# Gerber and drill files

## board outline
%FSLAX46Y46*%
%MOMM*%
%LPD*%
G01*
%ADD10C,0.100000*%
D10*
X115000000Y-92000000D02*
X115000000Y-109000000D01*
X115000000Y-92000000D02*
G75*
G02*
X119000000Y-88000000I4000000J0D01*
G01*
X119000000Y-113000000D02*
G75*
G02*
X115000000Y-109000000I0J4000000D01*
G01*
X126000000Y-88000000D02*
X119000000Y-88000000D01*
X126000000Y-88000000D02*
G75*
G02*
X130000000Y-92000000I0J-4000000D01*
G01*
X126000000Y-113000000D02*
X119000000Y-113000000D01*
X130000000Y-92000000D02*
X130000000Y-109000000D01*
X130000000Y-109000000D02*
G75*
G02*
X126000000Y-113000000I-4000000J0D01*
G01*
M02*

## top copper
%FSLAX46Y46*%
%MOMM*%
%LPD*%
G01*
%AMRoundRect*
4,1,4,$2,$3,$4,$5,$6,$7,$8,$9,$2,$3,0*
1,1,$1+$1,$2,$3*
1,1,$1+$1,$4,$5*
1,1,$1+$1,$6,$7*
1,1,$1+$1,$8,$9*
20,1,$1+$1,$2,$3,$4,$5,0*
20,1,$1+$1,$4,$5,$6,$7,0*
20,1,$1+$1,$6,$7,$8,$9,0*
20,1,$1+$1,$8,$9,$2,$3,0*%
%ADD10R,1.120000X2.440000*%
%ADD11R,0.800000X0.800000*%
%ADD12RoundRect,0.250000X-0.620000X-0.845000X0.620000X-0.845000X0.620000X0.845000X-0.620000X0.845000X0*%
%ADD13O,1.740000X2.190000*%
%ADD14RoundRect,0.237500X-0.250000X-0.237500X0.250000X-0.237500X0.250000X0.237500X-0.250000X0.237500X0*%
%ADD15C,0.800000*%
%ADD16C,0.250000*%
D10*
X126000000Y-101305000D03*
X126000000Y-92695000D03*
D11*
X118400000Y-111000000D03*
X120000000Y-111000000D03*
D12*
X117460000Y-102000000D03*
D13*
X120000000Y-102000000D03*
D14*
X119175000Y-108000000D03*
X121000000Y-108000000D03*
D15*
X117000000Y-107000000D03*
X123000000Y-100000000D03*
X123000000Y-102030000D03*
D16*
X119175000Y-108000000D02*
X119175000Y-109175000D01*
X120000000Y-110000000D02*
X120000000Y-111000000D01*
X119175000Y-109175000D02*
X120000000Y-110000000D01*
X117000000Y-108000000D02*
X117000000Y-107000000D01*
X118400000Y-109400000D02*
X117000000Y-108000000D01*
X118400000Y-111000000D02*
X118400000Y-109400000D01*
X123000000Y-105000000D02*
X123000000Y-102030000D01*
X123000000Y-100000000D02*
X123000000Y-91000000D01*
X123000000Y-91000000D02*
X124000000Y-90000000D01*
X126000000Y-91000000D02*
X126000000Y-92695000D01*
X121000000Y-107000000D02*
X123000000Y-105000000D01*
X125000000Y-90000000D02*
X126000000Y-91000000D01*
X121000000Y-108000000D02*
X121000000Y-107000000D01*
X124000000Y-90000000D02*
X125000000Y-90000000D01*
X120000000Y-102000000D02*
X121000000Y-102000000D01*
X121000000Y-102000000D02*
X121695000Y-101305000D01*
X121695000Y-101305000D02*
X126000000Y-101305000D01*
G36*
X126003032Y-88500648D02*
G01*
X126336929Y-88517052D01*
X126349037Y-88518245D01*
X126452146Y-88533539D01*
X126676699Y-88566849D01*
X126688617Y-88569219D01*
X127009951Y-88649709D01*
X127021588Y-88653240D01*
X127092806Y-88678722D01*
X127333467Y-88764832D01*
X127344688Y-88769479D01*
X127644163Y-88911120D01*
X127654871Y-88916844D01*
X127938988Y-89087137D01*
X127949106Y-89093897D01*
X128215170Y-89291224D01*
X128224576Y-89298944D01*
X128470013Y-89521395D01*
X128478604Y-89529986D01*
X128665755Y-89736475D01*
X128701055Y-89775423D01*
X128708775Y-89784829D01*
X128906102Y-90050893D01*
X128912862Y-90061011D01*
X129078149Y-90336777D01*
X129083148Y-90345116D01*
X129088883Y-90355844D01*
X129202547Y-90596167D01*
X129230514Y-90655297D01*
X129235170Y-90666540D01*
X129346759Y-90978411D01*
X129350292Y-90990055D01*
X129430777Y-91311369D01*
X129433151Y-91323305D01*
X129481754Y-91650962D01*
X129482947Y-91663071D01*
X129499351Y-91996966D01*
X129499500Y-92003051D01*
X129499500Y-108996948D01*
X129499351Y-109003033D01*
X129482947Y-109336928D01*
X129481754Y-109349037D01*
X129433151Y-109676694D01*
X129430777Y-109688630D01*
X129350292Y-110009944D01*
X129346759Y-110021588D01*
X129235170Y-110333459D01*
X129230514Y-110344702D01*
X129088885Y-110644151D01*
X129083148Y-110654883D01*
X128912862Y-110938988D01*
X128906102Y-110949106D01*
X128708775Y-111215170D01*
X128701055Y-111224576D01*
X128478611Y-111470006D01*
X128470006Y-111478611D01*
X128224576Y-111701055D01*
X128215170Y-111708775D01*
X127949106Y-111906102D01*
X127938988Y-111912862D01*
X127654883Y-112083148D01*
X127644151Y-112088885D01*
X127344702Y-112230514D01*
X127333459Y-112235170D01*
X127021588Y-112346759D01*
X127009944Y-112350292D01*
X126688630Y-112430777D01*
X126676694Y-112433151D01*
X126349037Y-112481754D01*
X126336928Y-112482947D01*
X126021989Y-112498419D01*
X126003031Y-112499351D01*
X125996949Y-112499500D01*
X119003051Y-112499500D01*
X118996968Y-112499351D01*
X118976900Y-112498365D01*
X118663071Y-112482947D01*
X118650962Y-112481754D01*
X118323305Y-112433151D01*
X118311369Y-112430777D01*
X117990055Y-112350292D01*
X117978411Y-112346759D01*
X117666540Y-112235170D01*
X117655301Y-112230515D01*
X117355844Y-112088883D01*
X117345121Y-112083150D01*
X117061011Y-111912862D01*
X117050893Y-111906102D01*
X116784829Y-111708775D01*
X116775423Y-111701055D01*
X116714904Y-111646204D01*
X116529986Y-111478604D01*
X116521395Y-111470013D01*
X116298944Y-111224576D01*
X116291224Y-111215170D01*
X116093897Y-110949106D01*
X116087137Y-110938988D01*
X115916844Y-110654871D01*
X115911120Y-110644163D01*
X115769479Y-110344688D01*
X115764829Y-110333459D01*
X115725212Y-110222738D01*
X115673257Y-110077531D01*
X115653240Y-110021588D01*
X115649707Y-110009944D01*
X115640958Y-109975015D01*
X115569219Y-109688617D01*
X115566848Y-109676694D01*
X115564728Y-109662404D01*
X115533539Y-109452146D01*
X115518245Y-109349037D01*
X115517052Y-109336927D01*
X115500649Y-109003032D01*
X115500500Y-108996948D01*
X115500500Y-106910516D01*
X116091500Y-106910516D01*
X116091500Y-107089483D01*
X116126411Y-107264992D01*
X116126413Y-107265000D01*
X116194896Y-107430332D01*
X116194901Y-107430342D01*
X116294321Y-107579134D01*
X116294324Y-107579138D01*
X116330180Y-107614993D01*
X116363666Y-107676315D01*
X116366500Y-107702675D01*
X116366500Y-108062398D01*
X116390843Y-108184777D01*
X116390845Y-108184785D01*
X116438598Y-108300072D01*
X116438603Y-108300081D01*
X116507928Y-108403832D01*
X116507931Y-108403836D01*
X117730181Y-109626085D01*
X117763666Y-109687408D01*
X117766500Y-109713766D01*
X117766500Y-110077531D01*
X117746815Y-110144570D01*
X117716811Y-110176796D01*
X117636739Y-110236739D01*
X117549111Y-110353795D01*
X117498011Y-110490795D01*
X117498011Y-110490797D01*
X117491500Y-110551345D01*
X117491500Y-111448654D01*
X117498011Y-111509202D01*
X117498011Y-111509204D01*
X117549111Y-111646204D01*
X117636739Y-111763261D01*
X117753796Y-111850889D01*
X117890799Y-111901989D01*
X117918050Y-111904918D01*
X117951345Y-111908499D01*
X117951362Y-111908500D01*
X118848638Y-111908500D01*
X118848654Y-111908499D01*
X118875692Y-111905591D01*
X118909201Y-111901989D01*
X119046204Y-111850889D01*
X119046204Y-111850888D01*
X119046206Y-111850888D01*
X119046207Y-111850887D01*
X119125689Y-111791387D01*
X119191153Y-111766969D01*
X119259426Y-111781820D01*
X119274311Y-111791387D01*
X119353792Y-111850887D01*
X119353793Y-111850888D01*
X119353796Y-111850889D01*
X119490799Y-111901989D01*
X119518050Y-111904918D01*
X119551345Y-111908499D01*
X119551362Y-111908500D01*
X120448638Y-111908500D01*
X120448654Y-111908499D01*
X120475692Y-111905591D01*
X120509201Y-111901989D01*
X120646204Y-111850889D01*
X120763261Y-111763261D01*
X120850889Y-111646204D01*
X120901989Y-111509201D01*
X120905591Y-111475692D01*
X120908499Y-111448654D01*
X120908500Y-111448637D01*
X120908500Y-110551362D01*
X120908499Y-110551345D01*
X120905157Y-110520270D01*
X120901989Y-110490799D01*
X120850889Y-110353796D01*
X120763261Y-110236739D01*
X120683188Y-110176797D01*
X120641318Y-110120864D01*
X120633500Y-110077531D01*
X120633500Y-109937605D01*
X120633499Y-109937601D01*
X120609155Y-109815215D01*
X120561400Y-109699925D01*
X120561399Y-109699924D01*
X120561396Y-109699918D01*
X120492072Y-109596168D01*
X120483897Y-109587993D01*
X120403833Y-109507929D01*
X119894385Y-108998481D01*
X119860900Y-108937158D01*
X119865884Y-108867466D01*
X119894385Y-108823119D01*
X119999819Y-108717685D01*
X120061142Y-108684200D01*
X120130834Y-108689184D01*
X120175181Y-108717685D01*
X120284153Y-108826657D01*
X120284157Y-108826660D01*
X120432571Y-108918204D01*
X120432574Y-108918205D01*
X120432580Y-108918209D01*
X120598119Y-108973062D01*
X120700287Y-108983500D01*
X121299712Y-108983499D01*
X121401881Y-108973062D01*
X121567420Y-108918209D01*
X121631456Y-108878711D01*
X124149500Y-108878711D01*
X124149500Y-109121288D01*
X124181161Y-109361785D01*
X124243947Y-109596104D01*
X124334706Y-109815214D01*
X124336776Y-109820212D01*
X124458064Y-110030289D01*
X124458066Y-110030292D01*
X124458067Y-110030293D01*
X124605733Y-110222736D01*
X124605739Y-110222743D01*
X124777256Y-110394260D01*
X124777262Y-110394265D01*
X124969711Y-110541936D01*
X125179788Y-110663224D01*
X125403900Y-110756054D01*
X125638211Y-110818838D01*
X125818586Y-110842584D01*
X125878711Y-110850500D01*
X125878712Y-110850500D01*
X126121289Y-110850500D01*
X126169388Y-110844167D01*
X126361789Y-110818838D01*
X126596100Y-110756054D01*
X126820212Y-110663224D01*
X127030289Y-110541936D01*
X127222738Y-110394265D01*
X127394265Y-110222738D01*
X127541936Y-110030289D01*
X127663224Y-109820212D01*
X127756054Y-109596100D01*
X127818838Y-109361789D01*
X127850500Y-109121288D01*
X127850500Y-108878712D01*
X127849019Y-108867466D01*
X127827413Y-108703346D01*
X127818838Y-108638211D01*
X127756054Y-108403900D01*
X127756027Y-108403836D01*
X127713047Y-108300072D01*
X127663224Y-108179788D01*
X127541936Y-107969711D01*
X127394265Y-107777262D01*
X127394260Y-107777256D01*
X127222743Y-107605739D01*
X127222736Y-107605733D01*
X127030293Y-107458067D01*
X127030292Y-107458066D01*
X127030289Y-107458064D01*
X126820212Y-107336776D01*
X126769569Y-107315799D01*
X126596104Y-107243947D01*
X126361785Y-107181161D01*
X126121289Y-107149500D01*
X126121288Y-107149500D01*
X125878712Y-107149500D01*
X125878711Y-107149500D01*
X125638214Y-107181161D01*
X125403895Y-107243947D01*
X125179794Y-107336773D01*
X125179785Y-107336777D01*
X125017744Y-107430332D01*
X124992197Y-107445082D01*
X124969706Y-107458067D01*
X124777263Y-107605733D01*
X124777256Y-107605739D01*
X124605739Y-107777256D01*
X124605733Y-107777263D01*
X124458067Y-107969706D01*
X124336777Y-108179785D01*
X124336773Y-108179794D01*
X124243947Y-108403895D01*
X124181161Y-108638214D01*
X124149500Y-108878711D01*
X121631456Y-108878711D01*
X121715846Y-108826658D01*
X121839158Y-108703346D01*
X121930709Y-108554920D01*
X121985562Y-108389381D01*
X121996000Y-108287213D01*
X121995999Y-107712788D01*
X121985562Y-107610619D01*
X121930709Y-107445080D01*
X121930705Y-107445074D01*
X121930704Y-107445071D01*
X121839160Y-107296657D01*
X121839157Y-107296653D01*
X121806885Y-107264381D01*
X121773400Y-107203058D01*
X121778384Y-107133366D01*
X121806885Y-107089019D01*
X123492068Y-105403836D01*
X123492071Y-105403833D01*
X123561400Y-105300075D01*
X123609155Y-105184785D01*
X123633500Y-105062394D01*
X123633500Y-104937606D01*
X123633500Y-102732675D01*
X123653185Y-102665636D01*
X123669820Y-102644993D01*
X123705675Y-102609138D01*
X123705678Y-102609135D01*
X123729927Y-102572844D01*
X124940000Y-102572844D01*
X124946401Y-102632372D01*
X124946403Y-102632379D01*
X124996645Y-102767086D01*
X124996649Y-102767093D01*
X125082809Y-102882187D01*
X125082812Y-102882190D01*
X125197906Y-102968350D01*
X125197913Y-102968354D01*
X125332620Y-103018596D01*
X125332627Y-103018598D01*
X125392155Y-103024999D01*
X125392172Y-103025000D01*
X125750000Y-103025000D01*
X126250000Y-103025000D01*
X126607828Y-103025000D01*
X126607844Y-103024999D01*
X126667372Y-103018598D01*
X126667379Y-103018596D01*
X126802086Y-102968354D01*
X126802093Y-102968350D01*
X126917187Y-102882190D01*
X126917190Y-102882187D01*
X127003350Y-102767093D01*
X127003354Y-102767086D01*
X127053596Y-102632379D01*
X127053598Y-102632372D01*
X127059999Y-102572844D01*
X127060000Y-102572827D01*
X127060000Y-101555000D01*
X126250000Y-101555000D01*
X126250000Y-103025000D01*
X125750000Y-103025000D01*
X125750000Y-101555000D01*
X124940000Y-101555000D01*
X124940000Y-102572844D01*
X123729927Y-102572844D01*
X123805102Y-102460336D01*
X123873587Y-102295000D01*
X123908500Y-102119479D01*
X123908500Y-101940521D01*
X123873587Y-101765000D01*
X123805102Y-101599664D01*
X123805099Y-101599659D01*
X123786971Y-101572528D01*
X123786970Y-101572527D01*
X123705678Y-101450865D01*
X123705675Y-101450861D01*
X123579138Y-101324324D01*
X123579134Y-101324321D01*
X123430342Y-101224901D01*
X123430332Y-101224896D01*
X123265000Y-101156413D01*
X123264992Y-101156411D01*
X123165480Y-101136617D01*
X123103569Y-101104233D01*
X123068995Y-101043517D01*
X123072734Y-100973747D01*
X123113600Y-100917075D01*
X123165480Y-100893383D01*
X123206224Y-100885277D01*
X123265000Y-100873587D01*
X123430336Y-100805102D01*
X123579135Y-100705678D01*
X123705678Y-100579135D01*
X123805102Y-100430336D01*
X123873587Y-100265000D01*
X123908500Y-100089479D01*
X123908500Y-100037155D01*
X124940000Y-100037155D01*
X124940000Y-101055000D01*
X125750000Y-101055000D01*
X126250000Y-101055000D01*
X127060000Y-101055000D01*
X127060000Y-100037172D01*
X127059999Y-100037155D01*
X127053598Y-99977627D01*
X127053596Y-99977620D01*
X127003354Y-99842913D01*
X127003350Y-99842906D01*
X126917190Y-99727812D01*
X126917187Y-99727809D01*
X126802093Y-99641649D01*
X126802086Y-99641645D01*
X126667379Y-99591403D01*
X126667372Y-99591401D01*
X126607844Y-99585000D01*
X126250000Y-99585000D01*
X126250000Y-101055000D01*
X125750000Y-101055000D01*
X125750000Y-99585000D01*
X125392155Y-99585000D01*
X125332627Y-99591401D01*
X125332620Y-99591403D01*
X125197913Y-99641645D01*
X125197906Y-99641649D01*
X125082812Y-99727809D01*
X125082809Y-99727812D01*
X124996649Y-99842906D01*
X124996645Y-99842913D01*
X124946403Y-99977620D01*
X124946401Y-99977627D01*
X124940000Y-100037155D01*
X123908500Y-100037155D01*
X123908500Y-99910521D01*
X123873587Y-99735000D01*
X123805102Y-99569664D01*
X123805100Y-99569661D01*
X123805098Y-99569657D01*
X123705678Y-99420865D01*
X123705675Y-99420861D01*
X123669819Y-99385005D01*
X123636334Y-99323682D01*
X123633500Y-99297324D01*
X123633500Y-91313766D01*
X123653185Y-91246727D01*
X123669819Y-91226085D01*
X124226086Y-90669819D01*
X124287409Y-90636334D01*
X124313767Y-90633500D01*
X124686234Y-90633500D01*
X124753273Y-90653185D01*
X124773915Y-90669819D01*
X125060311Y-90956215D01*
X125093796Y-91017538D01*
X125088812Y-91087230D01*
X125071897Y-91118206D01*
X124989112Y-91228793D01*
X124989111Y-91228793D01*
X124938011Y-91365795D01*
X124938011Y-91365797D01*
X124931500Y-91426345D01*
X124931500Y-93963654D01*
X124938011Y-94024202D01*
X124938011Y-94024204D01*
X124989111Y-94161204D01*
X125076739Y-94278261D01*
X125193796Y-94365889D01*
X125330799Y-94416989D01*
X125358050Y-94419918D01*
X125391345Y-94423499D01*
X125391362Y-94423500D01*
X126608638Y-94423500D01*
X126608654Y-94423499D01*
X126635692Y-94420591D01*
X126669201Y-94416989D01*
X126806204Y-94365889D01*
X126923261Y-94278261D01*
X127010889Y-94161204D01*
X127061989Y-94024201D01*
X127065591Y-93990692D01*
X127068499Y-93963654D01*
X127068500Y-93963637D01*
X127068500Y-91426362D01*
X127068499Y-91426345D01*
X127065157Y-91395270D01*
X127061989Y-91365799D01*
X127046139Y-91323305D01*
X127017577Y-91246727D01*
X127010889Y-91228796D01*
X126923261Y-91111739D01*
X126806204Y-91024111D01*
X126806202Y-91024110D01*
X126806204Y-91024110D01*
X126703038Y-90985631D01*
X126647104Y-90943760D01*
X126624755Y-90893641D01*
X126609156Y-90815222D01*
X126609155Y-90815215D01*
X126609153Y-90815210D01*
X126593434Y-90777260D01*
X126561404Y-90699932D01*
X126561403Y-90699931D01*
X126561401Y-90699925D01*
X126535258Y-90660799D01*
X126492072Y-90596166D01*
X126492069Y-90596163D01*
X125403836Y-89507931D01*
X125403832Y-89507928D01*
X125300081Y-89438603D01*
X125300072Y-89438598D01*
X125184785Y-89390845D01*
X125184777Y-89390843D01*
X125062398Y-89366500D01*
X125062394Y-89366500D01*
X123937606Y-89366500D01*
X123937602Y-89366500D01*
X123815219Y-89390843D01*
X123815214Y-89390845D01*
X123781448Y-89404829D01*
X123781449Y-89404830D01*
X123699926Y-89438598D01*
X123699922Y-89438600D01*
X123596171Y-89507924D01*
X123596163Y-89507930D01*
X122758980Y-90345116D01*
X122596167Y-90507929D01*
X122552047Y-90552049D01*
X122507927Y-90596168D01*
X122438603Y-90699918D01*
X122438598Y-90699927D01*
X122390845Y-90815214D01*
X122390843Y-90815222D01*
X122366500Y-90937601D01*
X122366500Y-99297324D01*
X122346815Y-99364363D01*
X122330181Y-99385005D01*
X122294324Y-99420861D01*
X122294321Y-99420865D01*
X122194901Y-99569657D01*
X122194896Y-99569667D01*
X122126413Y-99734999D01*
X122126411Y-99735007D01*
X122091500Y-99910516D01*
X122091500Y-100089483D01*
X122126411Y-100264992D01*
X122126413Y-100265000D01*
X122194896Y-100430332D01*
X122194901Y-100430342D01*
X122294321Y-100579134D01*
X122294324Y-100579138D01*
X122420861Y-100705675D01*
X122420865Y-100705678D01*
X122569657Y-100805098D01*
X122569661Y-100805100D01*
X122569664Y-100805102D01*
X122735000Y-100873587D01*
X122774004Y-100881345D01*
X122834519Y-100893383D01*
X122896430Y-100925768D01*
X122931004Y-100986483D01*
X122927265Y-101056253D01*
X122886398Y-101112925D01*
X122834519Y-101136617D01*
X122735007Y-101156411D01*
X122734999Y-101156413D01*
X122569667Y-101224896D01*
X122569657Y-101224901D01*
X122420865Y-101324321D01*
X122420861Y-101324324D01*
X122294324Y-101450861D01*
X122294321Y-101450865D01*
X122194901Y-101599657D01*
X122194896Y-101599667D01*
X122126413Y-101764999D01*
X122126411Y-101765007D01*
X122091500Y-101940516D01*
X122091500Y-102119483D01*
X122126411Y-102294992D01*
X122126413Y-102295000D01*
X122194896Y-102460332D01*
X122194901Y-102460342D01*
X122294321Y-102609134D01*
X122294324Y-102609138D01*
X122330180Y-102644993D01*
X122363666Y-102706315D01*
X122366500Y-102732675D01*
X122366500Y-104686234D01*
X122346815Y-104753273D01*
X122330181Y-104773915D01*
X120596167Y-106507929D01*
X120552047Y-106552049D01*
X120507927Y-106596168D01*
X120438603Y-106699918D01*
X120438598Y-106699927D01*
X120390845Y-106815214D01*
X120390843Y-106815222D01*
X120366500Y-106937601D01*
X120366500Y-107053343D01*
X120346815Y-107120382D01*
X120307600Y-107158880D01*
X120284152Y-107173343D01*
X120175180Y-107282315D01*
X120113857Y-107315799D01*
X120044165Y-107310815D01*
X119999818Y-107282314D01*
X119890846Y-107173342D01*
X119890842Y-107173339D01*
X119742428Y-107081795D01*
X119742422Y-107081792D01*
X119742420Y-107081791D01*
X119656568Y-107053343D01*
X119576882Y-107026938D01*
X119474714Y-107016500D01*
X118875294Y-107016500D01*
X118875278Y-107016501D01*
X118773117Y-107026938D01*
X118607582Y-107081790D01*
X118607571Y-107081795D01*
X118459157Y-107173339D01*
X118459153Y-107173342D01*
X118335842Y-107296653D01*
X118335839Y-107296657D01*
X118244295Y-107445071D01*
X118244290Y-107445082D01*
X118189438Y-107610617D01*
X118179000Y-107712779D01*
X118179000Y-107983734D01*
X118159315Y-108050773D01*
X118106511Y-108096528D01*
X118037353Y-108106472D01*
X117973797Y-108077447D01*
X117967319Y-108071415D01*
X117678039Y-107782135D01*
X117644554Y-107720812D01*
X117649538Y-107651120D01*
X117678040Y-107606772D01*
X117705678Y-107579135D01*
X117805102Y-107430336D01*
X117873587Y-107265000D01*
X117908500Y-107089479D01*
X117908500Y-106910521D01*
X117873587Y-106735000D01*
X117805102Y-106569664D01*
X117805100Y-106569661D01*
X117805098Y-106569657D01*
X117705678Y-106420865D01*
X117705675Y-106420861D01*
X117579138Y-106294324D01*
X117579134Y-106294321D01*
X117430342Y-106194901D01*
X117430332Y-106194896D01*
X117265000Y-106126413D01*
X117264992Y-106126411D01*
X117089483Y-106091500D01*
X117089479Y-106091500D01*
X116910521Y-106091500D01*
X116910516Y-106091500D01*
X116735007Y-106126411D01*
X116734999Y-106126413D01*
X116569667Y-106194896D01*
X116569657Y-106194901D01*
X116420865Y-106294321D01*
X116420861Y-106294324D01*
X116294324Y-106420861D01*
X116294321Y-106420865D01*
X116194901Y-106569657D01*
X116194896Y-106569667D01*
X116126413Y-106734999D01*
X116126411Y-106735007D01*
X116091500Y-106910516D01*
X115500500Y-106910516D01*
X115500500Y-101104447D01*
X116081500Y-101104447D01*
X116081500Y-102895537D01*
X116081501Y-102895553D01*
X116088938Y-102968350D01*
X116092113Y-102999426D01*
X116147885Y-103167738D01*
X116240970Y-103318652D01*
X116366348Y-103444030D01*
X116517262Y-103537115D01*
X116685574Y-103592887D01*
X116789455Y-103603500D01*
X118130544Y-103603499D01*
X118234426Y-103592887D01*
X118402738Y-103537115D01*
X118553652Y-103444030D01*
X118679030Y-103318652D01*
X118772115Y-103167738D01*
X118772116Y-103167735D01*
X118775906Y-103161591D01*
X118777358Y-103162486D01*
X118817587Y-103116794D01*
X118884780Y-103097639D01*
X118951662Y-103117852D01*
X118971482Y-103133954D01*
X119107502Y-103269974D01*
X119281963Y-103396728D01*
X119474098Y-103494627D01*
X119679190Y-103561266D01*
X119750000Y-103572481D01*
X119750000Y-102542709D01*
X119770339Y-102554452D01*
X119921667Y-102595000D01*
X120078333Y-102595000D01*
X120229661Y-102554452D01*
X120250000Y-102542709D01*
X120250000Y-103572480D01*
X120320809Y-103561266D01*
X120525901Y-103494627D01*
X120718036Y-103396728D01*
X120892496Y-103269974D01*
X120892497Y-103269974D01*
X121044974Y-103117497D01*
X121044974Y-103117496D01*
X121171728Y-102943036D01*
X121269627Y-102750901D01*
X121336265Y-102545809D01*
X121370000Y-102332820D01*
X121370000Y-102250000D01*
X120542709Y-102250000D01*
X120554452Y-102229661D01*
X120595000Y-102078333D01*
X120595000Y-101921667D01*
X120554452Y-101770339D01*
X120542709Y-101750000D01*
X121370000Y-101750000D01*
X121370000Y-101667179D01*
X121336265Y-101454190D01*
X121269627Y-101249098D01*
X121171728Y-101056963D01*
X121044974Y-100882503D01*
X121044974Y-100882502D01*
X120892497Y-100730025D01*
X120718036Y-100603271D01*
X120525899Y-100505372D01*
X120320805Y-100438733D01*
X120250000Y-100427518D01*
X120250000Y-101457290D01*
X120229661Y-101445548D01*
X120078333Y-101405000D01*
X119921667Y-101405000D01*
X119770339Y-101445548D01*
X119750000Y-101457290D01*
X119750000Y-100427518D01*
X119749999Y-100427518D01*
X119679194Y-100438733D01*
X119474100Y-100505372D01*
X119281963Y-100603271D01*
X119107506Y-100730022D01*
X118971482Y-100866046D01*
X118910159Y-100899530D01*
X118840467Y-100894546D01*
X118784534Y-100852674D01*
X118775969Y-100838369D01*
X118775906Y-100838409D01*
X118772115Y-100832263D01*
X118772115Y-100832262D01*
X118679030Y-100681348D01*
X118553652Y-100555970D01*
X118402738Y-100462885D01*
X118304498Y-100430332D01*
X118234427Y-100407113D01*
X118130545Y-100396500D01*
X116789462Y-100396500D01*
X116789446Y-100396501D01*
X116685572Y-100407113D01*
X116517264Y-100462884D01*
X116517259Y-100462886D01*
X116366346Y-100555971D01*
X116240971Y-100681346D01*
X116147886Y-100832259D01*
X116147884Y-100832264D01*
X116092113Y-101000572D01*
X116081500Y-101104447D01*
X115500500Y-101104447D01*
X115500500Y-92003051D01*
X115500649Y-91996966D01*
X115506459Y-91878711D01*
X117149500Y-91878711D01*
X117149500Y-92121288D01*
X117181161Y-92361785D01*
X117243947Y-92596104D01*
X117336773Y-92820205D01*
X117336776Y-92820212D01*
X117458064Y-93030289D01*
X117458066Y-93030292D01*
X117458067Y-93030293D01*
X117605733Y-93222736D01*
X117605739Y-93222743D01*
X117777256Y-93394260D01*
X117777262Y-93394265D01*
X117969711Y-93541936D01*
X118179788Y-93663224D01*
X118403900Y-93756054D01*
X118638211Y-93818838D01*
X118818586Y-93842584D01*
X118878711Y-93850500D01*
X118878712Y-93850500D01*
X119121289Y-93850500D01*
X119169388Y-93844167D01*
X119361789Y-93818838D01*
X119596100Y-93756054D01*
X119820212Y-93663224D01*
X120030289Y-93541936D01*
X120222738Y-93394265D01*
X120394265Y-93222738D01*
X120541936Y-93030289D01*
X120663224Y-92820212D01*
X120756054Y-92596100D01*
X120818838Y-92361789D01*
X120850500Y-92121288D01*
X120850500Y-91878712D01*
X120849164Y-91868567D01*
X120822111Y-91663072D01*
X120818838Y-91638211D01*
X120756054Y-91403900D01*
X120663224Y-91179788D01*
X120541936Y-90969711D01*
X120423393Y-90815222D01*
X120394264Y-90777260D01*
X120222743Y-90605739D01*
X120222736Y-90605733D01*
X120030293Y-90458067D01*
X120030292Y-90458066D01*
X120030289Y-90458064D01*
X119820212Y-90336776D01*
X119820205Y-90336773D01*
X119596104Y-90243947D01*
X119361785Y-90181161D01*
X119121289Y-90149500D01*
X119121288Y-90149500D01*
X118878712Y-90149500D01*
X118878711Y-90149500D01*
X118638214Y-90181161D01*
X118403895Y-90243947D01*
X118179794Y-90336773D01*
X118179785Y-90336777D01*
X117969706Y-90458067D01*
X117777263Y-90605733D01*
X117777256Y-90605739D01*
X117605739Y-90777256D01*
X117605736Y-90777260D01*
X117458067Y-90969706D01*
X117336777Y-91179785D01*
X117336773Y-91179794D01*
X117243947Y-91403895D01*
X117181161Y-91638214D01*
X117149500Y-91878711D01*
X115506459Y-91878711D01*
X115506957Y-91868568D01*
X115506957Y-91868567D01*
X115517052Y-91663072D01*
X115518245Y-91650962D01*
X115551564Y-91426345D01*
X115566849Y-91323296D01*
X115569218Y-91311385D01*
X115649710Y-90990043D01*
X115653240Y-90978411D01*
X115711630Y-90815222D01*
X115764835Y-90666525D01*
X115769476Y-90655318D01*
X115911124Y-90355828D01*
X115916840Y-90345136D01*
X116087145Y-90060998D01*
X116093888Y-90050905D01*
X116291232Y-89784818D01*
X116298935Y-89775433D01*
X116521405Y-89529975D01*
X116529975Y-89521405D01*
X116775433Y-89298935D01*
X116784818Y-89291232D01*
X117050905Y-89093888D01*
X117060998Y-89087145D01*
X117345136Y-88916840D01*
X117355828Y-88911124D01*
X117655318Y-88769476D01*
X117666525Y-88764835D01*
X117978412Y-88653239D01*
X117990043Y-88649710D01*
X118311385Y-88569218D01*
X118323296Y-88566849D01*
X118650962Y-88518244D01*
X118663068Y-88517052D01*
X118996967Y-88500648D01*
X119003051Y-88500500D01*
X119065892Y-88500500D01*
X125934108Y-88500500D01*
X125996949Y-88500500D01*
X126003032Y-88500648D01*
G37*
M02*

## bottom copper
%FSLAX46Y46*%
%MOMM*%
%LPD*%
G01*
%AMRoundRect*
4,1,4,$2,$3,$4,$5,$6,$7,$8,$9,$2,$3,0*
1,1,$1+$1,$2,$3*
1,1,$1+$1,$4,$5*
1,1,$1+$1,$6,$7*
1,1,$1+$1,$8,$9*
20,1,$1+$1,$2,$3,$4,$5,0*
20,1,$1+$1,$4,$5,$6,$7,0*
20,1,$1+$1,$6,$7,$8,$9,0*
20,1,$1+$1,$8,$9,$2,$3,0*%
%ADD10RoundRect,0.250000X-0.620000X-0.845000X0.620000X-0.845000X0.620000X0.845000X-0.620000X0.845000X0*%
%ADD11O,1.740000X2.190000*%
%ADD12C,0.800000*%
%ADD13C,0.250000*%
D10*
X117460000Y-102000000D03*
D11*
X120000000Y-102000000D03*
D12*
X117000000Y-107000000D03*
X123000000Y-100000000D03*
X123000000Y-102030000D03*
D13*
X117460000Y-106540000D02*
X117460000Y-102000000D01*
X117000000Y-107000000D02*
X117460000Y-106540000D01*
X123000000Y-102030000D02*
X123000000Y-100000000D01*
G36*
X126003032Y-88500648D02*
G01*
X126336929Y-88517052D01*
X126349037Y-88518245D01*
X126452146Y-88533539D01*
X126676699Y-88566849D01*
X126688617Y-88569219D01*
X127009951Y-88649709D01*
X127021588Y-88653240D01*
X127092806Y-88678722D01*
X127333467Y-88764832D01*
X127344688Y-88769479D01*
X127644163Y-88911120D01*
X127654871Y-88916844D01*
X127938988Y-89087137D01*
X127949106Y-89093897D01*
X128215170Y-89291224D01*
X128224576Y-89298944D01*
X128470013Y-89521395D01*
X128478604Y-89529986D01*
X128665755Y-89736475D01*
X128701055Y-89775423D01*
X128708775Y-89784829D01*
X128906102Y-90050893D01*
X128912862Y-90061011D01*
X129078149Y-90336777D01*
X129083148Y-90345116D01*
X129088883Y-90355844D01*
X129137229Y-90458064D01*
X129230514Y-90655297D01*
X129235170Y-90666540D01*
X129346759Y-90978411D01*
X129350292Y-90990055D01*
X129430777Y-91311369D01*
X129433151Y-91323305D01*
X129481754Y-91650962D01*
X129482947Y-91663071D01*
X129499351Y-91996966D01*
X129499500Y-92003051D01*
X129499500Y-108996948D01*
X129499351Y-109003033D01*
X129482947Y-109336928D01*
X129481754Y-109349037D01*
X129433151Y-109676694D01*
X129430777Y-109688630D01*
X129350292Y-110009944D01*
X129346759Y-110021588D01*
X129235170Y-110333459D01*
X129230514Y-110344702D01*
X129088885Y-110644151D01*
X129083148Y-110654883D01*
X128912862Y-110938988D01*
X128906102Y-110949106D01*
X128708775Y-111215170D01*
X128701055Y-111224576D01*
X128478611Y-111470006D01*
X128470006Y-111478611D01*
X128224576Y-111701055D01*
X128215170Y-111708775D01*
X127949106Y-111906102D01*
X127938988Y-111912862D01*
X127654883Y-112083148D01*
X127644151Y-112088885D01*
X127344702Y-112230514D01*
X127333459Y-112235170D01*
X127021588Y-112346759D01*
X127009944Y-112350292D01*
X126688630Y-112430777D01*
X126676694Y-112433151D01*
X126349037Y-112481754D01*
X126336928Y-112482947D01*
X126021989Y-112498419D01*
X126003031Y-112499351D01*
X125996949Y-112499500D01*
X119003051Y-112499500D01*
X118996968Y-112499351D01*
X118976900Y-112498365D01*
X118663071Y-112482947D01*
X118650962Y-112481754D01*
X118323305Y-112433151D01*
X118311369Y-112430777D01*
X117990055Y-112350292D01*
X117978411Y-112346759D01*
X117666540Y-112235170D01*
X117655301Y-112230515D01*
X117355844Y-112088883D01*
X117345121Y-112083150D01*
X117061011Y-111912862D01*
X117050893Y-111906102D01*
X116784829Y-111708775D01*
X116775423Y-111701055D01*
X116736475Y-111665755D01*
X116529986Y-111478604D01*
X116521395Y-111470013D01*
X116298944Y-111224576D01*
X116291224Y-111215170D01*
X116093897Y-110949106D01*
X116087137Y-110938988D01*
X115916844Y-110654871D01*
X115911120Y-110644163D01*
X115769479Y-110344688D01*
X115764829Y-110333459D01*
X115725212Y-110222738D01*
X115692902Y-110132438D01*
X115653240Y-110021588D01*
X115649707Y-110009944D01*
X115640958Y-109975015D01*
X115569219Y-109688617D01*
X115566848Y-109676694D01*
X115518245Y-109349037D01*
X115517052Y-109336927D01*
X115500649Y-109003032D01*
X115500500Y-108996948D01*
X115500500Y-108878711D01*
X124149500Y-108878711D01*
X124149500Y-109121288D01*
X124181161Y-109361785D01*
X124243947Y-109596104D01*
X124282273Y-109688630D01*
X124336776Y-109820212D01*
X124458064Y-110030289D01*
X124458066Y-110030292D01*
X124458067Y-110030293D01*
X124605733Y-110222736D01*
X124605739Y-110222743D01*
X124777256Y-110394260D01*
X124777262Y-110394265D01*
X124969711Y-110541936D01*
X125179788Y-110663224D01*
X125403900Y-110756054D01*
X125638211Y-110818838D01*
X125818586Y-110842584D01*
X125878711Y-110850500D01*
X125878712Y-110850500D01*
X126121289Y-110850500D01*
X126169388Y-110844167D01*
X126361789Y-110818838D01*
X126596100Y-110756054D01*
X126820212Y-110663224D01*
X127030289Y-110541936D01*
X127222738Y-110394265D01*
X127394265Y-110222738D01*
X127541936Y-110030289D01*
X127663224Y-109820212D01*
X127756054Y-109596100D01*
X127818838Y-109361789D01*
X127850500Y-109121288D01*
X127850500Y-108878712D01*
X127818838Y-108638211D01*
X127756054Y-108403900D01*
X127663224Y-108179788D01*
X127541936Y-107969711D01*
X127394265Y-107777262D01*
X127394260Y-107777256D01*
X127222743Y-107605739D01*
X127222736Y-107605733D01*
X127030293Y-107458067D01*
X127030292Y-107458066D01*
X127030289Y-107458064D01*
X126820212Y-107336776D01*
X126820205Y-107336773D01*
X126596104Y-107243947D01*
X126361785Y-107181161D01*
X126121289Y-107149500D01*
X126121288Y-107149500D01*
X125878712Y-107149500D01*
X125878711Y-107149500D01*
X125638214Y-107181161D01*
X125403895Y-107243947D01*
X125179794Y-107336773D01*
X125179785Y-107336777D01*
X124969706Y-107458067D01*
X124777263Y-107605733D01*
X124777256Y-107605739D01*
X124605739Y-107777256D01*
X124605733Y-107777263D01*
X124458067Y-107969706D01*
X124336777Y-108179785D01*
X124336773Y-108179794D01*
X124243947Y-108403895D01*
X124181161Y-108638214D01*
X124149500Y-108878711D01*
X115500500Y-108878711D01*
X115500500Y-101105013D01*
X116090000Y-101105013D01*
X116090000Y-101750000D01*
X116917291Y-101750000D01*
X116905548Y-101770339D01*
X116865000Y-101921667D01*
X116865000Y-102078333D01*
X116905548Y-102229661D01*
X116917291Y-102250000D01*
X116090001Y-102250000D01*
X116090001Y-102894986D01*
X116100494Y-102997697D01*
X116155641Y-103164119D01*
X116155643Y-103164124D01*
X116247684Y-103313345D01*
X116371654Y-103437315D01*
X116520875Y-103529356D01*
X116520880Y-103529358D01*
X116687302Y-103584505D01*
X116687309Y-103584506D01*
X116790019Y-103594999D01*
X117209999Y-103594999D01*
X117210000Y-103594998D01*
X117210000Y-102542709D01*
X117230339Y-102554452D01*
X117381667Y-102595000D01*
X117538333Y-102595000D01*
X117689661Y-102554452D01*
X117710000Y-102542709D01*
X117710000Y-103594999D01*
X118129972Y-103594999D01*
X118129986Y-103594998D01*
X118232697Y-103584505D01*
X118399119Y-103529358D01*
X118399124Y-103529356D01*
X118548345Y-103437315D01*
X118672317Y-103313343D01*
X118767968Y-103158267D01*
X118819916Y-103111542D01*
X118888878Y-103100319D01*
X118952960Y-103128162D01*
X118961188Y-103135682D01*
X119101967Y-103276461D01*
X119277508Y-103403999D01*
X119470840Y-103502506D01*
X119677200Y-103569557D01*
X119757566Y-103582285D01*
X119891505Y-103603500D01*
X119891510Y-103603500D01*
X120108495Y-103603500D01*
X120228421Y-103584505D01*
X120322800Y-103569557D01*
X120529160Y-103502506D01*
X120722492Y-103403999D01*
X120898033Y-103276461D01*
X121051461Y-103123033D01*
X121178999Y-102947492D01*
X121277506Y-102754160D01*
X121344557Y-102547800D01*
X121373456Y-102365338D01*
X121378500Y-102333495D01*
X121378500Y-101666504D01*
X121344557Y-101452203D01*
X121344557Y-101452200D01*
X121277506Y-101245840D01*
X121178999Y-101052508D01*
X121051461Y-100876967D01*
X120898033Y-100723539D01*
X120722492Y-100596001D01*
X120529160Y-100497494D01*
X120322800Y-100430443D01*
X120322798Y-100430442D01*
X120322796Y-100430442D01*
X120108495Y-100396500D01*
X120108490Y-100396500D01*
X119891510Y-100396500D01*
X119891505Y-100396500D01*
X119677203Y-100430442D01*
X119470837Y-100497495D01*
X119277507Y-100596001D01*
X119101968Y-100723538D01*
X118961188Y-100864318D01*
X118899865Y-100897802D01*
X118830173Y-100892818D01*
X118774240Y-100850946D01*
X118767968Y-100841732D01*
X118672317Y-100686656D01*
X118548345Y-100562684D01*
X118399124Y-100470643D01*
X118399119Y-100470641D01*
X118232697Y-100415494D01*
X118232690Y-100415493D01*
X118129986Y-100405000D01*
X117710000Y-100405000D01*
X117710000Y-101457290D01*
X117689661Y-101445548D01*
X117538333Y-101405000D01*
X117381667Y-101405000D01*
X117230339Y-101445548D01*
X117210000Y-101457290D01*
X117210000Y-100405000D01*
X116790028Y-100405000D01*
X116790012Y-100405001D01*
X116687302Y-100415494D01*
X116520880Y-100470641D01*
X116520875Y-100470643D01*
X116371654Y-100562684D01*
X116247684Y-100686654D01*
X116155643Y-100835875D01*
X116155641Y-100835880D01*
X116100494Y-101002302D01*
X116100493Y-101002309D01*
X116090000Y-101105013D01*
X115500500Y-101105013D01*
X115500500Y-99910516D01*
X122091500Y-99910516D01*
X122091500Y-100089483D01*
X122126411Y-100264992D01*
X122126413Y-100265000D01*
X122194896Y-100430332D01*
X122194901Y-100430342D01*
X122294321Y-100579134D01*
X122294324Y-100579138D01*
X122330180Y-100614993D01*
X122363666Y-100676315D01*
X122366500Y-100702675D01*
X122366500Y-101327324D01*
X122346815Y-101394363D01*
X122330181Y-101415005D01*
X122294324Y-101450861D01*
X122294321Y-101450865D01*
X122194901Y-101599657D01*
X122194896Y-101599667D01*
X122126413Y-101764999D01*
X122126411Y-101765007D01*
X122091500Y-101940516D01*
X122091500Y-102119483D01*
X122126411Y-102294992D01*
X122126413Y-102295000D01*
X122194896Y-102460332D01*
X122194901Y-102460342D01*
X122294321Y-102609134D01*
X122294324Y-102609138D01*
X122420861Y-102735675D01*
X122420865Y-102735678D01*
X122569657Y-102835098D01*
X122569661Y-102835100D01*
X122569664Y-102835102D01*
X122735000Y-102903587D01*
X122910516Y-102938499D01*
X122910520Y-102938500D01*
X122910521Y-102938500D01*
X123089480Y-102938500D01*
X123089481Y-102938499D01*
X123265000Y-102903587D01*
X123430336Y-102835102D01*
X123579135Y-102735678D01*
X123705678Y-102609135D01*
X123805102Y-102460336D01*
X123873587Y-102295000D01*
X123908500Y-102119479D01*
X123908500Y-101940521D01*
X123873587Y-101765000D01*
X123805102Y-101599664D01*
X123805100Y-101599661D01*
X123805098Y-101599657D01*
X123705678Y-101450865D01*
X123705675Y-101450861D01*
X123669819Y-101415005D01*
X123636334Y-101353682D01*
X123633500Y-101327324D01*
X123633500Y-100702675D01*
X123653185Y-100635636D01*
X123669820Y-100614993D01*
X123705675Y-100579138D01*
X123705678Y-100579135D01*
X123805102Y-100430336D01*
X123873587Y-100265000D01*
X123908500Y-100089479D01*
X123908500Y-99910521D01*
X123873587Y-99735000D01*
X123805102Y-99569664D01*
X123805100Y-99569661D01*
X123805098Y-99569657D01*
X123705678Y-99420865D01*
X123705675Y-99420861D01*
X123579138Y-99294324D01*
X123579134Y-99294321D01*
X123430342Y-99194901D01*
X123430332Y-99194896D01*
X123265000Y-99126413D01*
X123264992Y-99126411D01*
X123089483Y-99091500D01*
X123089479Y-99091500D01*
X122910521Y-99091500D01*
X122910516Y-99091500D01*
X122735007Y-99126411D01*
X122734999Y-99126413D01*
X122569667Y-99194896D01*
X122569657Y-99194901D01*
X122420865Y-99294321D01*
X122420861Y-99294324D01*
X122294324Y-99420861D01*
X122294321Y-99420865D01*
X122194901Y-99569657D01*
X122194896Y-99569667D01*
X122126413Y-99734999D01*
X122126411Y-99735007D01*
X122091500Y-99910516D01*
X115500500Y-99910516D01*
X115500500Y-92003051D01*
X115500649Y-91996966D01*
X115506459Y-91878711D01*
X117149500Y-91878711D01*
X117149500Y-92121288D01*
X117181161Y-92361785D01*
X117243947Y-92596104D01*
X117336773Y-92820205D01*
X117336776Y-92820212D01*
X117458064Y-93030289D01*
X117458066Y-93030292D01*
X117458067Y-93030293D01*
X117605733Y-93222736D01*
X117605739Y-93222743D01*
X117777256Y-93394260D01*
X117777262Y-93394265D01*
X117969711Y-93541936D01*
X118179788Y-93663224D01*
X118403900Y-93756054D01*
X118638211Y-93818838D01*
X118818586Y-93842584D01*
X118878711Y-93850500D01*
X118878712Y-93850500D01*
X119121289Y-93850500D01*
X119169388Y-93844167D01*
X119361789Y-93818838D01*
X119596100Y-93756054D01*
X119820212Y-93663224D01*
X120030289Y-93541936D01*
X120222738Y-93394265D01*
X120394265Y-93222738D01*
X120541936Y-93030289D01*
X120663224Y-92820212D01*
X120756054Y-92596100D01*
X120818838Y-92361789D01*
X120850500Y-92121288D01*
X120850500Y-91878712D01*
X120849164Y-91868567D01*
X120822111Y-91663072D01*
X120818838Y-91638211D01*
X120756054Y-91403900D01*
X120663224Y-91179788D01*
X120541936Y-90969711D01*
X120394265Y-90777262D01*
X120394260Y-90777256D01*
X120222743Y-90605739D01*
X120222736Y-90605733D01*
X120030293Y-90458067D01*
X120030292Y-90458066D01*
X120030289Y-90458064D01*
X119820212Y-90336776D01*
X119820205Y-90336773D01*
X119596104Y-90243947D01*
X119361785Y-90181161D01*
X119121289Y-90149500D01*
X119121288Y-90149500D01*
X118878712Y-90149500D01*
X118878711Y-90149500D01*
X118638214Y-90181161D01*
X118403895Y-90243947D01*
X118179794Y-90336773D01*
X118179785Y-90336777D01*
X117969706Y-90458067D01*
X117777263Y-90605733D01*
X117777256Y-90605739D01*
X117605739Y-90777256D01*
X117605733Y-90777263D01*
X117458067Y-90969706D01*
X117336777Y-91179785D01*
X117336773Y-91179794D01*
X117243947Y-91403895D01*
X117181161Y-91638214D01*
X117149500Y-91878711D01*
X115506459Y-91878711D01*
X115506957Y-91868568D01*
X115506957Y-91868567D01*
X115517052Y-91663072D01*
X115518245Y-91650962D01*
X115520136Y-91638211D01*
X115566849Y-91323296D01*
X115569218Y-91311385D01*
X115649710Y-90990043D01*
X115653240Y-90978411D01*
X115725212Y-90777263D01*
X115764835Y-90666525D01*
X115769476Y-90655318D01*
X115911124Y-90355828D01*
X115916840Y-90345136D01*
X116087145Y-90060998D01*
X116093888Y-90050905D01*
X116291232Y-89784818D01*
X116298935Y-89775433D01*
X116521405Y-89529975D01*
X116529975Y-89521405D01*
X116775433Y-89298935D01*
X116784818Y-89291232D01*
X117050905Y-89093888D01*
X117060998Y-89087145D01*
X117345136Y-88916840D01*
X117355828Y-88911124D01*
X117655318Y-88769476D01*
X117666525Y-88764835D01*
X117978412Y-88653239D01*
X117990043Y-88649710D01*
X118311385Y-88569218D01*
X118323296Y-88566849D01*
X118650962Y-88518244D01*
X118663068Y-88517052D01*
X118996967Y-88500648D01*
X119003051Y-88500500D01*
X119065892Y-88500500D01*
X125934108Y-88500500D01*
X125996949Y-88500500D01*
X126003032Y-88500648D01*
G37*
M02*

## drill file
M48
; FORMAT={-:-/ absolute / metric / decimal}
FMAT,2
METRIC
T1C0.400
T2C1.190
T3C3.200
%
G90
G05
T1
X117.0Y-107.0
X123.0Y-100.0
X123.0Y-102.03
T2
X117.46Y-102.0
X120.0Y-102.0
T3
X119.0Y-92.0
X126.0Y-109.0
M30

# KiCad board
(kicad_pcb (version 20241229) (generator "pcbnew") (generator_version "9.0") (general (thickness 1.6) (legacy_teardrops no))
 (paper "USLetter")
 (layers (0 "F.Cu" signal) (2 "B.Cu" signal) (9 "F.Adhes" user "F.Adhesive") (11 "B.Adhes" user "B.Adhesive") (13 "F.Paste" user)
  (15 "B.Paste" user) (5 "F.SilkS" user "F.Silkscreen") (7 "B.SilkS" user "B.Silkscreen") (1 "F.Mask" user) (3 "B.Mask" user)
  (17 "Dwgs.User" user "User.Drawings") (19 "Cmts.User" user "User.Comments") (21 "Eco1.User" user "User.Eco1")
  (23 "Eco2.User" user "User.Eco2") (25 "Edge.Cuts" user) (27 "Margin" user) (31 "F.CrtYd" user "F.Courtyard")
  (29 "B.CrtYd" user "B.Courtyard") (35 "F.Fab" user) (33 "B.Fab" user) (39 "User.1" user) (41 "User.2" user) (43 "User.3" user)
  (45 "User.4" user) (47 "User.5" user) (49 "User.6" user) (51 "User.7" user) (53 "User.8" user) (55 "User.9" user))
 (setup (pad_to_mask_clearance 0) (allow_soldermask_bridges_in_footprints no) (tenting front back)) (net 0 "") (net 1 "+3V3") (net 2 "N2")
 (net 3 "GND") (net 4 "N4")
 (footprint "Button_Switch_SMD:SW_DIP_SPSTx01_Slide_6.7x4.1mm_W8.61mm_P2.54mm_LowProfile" (layer "F.Cu") (at 126 97 90)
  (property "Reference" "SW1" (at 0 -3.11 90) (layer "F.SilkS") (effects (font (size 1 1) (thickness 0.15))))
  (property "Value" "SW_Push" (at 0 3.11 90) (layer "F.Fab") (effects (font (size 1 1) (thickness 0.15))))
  (pad "1" smd rect (at -4.305 0 90) (size 2.44 1.12) (layers "F.Cu" "F.Mask" "F.Paste") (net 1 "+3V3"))
  (pad "2" smd rect (at 4.305 0 90) (size 2.44 1.12) (layers "F.Cu" "F.Mask" "F.Paste") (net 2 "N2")))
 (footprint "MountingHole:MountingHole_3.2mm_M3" (layer "F.Cu") (at 126 109)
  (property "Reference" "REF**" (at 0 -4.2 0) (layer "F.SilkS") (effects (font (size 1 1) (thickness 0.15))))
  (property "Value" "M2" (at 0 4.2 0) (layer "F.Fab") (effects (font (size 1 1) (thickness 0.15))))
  (pad "" np_thru_hole circle (at 0 0) (size 3.2 3.2) (drill 3.2) (layers "*.Cu" "*.Mask")))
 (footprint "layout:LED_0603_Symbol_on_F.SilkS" (layer "F.Cu") (at 119.2 111)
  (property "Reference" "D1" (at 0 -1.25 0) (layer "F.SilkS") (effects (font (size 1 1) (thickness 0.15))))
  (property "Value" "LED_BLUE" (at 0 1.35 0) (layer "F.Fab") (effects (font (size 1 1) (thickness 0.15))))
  (pad "1" smd rect (at -0.8 0 180) (size 0.8 0.8) (layers "F.Cu" "F.Mask" "F.Paste") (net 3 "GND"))
  (pad "2" smd rect (at 0.8 0 180) (size 0.8 0.8) (layers "F.Cu" "F.Mask" "F.Paste") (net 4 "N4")))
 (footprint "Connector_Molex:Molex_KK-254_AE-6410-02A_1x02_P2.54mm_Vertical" (layer "F.Cu") (at 117.46 102)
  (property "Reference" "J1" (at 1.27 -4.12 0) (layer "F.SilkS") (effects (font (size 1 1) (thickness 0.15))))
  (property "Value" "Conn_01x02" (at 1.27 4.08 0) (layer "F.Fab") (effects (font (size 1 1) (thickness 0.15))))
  (pad "1" thru_hole roundrect (at 0 0) (size 1.74 2.19) (drill 1.19) (layers "*.Cu" "*.Mask") (remove_unused_layers no)
   (roundrect_rratio 0.143678) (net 3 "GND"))
  (pad "2" thru_hole oval (at 2.54 0) (size 1.74 2.19) (drill 1.19) (layers "*.Cu" "*.Mask") (remove_unused_layers no) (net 1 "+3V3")))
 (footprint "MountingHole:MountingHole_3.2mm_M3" (layer "F.Cu") (at 119 92)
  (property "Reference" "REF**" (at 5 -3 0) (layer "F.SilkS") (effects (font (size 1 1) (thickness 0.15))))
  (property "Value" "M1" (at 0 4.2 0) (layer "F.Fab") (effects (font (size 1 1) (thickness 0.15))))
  (pad "" np_thru_hole circle (at 0 0) (size 3.2 3.2) (drill 3.2) (layers "*.Cu" "*.Mask")))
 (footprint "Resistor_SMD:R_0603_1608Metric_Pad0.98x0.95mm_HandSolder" (layer "F.Cu") (at 120.0875 108)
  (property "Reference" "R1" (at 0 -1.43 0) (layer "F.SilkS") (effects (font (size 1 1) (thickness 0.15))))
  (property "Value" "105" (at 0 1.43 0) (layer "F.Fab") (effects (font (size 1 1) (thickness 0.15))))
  (pad "1" smd roundrect (at -0.9125 0) (size 0.975 0.95) (layers "F.Cu" "F.Mask" "F.Paste") (roundrect_rratio 0.25) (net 4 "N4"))
  (pad "2" smd roundrect (at 0.9125 0) (size 0.975 0.95) (layers "F.Cu" "F.Mask" "F.Paste") (roundrect_rratio 0.25) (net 2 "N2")))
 (gr_line (start 115 92) (end 115 109) (stroke (width 0.1) (type default)) (layer "Edge.Cuts"))
 (gr_arc (start 115 92) (mid 116.171573 89.171573) (end 119 88) (stroke (width 0.1) (type default)) (layer "Edge.Cuts"))
 (gr_arc (start 119 113) (mid 116.171573 111.828427) (end 115 109) (stroke (width 0.1) (type default)) (layer "Edge.Cuts"))
 (gr_line (start 126 88) (end 119 88) (stroke (width 0.1) (type default)) (layer "Edge.Cuts"))
 (gr_arc (start 126 88) (mid 128.828427 89.171573) (end 130 92) (stroke (width 0.1) (type default)) (layer "Edge.Cuts"))
 (gr_line (start 126 113) (end 119 113) (stroke (width 0.1) (type default)) (layer "Edge.Cuts"))
 (gr_line (start 130 92) (end 130 109) (stroke (width 0.1) (type default)) (layer "Edge.Cuts"))
 (gr_arc (start 130 109) (mid 128.828427 111.828427) (end 126 113) (stroke (width 0.1) (type default)) (layer "Edge.Cuts"))
 (segment (start 119.175 108) (end 119.175 109.175) (width 0.25) (layer "F.Cu") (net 4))
 (segment (start 120 110) (end 120 111) (width 0.25) (layer "F.Cu") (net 4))
 (segment (start 119.175 109.175) (end 120 110) (width 0.25) (layer "F.Cu") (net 4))
 (segment (start 117 108) (end 117 107) (width 0.25) (layer "F.Cu") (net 3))
 (segment (start 118.4 109.4) (end 117 108) (width 0.25) (layer "F.Cu") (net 3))
 (segment (start 118.4 111) (end 118.4 109.4) (width 0.25) (layer "F.Cu") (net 3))
 (via (at 117 107) (size 0.8) (drill 0.4) (layers "F.Cu" "B.Cu") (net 3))
 (segment (start 117.46 106.54) (end 117.46 102) (width 0.25) (layer "B.Cu") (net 3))
 (segment (start 117 107) (end 117.46 106.54) (width 0.25) (layer "B.Cu") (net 3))
 (segment (start 123 105) (end 123 102.03) (width 0.25) (layer "F.Cu") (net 2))
 (segment (start 123 100) (end 123 91) (width 0.25) (layer "F.Cu") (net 2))
 (segment (start 123 91) (end 124 90) (width 0.25) (layer "F.Cu") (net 2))
 (segment (start 126 91) (end 126 92.695) (width 0.25) (layer "F.Cu") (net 2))
 (segment (start 121 107) (end 123 105) (width 0.25) (layer "F.Cu") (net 2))
 (segment (start 125 90) (end 126 91) (width 0.25) (layer "F.Cu") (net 2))
 (segment (start 121 108) (end 121 107) (width 0.25) (layer "F.Cu") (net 2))
 (segment (start 124 90) (end 125 90) (width 0.25) (layer "F.Cu") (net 2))
 (via (at 123 100) (size 0.8) (drill 0.4) (layers "F.Cu" "B.Cu") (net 2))
 (via (at 123 102.03) (size 0.8) (drill 0.4) (layers "F.Cu" "B.Cu") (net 2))
 (segment (start 123 102.03) (end 123 100) (width 0.25) (layer "B.Cu") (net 2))
 (segment (start 120 102) (end 121 102) (width 0.25) (layer "F.Cu") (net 1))
 (segment (start 121 102) (end 121.695 101.305) (width 0.25) (layer "F.Cu") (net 1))
 (segment (start 121.695 101.305) (end 126 101.305) (width 0.25) (layer "F.Cu") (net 1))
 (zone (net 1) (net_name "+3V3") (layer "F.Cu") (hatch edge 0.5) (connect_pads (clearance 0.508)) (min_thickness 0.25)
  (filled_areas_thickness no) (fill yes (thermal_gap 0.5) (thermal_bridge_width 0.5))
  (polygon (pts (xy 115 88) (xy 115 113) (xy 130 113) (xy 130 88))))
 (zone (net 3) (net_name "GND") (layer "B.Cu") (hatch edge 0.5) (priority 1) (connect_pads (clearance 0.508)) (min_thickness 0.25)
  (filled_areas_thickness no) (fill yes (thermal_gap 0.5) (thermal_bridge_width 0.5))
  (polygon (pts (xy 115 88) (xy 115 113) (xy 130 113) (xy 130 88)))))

